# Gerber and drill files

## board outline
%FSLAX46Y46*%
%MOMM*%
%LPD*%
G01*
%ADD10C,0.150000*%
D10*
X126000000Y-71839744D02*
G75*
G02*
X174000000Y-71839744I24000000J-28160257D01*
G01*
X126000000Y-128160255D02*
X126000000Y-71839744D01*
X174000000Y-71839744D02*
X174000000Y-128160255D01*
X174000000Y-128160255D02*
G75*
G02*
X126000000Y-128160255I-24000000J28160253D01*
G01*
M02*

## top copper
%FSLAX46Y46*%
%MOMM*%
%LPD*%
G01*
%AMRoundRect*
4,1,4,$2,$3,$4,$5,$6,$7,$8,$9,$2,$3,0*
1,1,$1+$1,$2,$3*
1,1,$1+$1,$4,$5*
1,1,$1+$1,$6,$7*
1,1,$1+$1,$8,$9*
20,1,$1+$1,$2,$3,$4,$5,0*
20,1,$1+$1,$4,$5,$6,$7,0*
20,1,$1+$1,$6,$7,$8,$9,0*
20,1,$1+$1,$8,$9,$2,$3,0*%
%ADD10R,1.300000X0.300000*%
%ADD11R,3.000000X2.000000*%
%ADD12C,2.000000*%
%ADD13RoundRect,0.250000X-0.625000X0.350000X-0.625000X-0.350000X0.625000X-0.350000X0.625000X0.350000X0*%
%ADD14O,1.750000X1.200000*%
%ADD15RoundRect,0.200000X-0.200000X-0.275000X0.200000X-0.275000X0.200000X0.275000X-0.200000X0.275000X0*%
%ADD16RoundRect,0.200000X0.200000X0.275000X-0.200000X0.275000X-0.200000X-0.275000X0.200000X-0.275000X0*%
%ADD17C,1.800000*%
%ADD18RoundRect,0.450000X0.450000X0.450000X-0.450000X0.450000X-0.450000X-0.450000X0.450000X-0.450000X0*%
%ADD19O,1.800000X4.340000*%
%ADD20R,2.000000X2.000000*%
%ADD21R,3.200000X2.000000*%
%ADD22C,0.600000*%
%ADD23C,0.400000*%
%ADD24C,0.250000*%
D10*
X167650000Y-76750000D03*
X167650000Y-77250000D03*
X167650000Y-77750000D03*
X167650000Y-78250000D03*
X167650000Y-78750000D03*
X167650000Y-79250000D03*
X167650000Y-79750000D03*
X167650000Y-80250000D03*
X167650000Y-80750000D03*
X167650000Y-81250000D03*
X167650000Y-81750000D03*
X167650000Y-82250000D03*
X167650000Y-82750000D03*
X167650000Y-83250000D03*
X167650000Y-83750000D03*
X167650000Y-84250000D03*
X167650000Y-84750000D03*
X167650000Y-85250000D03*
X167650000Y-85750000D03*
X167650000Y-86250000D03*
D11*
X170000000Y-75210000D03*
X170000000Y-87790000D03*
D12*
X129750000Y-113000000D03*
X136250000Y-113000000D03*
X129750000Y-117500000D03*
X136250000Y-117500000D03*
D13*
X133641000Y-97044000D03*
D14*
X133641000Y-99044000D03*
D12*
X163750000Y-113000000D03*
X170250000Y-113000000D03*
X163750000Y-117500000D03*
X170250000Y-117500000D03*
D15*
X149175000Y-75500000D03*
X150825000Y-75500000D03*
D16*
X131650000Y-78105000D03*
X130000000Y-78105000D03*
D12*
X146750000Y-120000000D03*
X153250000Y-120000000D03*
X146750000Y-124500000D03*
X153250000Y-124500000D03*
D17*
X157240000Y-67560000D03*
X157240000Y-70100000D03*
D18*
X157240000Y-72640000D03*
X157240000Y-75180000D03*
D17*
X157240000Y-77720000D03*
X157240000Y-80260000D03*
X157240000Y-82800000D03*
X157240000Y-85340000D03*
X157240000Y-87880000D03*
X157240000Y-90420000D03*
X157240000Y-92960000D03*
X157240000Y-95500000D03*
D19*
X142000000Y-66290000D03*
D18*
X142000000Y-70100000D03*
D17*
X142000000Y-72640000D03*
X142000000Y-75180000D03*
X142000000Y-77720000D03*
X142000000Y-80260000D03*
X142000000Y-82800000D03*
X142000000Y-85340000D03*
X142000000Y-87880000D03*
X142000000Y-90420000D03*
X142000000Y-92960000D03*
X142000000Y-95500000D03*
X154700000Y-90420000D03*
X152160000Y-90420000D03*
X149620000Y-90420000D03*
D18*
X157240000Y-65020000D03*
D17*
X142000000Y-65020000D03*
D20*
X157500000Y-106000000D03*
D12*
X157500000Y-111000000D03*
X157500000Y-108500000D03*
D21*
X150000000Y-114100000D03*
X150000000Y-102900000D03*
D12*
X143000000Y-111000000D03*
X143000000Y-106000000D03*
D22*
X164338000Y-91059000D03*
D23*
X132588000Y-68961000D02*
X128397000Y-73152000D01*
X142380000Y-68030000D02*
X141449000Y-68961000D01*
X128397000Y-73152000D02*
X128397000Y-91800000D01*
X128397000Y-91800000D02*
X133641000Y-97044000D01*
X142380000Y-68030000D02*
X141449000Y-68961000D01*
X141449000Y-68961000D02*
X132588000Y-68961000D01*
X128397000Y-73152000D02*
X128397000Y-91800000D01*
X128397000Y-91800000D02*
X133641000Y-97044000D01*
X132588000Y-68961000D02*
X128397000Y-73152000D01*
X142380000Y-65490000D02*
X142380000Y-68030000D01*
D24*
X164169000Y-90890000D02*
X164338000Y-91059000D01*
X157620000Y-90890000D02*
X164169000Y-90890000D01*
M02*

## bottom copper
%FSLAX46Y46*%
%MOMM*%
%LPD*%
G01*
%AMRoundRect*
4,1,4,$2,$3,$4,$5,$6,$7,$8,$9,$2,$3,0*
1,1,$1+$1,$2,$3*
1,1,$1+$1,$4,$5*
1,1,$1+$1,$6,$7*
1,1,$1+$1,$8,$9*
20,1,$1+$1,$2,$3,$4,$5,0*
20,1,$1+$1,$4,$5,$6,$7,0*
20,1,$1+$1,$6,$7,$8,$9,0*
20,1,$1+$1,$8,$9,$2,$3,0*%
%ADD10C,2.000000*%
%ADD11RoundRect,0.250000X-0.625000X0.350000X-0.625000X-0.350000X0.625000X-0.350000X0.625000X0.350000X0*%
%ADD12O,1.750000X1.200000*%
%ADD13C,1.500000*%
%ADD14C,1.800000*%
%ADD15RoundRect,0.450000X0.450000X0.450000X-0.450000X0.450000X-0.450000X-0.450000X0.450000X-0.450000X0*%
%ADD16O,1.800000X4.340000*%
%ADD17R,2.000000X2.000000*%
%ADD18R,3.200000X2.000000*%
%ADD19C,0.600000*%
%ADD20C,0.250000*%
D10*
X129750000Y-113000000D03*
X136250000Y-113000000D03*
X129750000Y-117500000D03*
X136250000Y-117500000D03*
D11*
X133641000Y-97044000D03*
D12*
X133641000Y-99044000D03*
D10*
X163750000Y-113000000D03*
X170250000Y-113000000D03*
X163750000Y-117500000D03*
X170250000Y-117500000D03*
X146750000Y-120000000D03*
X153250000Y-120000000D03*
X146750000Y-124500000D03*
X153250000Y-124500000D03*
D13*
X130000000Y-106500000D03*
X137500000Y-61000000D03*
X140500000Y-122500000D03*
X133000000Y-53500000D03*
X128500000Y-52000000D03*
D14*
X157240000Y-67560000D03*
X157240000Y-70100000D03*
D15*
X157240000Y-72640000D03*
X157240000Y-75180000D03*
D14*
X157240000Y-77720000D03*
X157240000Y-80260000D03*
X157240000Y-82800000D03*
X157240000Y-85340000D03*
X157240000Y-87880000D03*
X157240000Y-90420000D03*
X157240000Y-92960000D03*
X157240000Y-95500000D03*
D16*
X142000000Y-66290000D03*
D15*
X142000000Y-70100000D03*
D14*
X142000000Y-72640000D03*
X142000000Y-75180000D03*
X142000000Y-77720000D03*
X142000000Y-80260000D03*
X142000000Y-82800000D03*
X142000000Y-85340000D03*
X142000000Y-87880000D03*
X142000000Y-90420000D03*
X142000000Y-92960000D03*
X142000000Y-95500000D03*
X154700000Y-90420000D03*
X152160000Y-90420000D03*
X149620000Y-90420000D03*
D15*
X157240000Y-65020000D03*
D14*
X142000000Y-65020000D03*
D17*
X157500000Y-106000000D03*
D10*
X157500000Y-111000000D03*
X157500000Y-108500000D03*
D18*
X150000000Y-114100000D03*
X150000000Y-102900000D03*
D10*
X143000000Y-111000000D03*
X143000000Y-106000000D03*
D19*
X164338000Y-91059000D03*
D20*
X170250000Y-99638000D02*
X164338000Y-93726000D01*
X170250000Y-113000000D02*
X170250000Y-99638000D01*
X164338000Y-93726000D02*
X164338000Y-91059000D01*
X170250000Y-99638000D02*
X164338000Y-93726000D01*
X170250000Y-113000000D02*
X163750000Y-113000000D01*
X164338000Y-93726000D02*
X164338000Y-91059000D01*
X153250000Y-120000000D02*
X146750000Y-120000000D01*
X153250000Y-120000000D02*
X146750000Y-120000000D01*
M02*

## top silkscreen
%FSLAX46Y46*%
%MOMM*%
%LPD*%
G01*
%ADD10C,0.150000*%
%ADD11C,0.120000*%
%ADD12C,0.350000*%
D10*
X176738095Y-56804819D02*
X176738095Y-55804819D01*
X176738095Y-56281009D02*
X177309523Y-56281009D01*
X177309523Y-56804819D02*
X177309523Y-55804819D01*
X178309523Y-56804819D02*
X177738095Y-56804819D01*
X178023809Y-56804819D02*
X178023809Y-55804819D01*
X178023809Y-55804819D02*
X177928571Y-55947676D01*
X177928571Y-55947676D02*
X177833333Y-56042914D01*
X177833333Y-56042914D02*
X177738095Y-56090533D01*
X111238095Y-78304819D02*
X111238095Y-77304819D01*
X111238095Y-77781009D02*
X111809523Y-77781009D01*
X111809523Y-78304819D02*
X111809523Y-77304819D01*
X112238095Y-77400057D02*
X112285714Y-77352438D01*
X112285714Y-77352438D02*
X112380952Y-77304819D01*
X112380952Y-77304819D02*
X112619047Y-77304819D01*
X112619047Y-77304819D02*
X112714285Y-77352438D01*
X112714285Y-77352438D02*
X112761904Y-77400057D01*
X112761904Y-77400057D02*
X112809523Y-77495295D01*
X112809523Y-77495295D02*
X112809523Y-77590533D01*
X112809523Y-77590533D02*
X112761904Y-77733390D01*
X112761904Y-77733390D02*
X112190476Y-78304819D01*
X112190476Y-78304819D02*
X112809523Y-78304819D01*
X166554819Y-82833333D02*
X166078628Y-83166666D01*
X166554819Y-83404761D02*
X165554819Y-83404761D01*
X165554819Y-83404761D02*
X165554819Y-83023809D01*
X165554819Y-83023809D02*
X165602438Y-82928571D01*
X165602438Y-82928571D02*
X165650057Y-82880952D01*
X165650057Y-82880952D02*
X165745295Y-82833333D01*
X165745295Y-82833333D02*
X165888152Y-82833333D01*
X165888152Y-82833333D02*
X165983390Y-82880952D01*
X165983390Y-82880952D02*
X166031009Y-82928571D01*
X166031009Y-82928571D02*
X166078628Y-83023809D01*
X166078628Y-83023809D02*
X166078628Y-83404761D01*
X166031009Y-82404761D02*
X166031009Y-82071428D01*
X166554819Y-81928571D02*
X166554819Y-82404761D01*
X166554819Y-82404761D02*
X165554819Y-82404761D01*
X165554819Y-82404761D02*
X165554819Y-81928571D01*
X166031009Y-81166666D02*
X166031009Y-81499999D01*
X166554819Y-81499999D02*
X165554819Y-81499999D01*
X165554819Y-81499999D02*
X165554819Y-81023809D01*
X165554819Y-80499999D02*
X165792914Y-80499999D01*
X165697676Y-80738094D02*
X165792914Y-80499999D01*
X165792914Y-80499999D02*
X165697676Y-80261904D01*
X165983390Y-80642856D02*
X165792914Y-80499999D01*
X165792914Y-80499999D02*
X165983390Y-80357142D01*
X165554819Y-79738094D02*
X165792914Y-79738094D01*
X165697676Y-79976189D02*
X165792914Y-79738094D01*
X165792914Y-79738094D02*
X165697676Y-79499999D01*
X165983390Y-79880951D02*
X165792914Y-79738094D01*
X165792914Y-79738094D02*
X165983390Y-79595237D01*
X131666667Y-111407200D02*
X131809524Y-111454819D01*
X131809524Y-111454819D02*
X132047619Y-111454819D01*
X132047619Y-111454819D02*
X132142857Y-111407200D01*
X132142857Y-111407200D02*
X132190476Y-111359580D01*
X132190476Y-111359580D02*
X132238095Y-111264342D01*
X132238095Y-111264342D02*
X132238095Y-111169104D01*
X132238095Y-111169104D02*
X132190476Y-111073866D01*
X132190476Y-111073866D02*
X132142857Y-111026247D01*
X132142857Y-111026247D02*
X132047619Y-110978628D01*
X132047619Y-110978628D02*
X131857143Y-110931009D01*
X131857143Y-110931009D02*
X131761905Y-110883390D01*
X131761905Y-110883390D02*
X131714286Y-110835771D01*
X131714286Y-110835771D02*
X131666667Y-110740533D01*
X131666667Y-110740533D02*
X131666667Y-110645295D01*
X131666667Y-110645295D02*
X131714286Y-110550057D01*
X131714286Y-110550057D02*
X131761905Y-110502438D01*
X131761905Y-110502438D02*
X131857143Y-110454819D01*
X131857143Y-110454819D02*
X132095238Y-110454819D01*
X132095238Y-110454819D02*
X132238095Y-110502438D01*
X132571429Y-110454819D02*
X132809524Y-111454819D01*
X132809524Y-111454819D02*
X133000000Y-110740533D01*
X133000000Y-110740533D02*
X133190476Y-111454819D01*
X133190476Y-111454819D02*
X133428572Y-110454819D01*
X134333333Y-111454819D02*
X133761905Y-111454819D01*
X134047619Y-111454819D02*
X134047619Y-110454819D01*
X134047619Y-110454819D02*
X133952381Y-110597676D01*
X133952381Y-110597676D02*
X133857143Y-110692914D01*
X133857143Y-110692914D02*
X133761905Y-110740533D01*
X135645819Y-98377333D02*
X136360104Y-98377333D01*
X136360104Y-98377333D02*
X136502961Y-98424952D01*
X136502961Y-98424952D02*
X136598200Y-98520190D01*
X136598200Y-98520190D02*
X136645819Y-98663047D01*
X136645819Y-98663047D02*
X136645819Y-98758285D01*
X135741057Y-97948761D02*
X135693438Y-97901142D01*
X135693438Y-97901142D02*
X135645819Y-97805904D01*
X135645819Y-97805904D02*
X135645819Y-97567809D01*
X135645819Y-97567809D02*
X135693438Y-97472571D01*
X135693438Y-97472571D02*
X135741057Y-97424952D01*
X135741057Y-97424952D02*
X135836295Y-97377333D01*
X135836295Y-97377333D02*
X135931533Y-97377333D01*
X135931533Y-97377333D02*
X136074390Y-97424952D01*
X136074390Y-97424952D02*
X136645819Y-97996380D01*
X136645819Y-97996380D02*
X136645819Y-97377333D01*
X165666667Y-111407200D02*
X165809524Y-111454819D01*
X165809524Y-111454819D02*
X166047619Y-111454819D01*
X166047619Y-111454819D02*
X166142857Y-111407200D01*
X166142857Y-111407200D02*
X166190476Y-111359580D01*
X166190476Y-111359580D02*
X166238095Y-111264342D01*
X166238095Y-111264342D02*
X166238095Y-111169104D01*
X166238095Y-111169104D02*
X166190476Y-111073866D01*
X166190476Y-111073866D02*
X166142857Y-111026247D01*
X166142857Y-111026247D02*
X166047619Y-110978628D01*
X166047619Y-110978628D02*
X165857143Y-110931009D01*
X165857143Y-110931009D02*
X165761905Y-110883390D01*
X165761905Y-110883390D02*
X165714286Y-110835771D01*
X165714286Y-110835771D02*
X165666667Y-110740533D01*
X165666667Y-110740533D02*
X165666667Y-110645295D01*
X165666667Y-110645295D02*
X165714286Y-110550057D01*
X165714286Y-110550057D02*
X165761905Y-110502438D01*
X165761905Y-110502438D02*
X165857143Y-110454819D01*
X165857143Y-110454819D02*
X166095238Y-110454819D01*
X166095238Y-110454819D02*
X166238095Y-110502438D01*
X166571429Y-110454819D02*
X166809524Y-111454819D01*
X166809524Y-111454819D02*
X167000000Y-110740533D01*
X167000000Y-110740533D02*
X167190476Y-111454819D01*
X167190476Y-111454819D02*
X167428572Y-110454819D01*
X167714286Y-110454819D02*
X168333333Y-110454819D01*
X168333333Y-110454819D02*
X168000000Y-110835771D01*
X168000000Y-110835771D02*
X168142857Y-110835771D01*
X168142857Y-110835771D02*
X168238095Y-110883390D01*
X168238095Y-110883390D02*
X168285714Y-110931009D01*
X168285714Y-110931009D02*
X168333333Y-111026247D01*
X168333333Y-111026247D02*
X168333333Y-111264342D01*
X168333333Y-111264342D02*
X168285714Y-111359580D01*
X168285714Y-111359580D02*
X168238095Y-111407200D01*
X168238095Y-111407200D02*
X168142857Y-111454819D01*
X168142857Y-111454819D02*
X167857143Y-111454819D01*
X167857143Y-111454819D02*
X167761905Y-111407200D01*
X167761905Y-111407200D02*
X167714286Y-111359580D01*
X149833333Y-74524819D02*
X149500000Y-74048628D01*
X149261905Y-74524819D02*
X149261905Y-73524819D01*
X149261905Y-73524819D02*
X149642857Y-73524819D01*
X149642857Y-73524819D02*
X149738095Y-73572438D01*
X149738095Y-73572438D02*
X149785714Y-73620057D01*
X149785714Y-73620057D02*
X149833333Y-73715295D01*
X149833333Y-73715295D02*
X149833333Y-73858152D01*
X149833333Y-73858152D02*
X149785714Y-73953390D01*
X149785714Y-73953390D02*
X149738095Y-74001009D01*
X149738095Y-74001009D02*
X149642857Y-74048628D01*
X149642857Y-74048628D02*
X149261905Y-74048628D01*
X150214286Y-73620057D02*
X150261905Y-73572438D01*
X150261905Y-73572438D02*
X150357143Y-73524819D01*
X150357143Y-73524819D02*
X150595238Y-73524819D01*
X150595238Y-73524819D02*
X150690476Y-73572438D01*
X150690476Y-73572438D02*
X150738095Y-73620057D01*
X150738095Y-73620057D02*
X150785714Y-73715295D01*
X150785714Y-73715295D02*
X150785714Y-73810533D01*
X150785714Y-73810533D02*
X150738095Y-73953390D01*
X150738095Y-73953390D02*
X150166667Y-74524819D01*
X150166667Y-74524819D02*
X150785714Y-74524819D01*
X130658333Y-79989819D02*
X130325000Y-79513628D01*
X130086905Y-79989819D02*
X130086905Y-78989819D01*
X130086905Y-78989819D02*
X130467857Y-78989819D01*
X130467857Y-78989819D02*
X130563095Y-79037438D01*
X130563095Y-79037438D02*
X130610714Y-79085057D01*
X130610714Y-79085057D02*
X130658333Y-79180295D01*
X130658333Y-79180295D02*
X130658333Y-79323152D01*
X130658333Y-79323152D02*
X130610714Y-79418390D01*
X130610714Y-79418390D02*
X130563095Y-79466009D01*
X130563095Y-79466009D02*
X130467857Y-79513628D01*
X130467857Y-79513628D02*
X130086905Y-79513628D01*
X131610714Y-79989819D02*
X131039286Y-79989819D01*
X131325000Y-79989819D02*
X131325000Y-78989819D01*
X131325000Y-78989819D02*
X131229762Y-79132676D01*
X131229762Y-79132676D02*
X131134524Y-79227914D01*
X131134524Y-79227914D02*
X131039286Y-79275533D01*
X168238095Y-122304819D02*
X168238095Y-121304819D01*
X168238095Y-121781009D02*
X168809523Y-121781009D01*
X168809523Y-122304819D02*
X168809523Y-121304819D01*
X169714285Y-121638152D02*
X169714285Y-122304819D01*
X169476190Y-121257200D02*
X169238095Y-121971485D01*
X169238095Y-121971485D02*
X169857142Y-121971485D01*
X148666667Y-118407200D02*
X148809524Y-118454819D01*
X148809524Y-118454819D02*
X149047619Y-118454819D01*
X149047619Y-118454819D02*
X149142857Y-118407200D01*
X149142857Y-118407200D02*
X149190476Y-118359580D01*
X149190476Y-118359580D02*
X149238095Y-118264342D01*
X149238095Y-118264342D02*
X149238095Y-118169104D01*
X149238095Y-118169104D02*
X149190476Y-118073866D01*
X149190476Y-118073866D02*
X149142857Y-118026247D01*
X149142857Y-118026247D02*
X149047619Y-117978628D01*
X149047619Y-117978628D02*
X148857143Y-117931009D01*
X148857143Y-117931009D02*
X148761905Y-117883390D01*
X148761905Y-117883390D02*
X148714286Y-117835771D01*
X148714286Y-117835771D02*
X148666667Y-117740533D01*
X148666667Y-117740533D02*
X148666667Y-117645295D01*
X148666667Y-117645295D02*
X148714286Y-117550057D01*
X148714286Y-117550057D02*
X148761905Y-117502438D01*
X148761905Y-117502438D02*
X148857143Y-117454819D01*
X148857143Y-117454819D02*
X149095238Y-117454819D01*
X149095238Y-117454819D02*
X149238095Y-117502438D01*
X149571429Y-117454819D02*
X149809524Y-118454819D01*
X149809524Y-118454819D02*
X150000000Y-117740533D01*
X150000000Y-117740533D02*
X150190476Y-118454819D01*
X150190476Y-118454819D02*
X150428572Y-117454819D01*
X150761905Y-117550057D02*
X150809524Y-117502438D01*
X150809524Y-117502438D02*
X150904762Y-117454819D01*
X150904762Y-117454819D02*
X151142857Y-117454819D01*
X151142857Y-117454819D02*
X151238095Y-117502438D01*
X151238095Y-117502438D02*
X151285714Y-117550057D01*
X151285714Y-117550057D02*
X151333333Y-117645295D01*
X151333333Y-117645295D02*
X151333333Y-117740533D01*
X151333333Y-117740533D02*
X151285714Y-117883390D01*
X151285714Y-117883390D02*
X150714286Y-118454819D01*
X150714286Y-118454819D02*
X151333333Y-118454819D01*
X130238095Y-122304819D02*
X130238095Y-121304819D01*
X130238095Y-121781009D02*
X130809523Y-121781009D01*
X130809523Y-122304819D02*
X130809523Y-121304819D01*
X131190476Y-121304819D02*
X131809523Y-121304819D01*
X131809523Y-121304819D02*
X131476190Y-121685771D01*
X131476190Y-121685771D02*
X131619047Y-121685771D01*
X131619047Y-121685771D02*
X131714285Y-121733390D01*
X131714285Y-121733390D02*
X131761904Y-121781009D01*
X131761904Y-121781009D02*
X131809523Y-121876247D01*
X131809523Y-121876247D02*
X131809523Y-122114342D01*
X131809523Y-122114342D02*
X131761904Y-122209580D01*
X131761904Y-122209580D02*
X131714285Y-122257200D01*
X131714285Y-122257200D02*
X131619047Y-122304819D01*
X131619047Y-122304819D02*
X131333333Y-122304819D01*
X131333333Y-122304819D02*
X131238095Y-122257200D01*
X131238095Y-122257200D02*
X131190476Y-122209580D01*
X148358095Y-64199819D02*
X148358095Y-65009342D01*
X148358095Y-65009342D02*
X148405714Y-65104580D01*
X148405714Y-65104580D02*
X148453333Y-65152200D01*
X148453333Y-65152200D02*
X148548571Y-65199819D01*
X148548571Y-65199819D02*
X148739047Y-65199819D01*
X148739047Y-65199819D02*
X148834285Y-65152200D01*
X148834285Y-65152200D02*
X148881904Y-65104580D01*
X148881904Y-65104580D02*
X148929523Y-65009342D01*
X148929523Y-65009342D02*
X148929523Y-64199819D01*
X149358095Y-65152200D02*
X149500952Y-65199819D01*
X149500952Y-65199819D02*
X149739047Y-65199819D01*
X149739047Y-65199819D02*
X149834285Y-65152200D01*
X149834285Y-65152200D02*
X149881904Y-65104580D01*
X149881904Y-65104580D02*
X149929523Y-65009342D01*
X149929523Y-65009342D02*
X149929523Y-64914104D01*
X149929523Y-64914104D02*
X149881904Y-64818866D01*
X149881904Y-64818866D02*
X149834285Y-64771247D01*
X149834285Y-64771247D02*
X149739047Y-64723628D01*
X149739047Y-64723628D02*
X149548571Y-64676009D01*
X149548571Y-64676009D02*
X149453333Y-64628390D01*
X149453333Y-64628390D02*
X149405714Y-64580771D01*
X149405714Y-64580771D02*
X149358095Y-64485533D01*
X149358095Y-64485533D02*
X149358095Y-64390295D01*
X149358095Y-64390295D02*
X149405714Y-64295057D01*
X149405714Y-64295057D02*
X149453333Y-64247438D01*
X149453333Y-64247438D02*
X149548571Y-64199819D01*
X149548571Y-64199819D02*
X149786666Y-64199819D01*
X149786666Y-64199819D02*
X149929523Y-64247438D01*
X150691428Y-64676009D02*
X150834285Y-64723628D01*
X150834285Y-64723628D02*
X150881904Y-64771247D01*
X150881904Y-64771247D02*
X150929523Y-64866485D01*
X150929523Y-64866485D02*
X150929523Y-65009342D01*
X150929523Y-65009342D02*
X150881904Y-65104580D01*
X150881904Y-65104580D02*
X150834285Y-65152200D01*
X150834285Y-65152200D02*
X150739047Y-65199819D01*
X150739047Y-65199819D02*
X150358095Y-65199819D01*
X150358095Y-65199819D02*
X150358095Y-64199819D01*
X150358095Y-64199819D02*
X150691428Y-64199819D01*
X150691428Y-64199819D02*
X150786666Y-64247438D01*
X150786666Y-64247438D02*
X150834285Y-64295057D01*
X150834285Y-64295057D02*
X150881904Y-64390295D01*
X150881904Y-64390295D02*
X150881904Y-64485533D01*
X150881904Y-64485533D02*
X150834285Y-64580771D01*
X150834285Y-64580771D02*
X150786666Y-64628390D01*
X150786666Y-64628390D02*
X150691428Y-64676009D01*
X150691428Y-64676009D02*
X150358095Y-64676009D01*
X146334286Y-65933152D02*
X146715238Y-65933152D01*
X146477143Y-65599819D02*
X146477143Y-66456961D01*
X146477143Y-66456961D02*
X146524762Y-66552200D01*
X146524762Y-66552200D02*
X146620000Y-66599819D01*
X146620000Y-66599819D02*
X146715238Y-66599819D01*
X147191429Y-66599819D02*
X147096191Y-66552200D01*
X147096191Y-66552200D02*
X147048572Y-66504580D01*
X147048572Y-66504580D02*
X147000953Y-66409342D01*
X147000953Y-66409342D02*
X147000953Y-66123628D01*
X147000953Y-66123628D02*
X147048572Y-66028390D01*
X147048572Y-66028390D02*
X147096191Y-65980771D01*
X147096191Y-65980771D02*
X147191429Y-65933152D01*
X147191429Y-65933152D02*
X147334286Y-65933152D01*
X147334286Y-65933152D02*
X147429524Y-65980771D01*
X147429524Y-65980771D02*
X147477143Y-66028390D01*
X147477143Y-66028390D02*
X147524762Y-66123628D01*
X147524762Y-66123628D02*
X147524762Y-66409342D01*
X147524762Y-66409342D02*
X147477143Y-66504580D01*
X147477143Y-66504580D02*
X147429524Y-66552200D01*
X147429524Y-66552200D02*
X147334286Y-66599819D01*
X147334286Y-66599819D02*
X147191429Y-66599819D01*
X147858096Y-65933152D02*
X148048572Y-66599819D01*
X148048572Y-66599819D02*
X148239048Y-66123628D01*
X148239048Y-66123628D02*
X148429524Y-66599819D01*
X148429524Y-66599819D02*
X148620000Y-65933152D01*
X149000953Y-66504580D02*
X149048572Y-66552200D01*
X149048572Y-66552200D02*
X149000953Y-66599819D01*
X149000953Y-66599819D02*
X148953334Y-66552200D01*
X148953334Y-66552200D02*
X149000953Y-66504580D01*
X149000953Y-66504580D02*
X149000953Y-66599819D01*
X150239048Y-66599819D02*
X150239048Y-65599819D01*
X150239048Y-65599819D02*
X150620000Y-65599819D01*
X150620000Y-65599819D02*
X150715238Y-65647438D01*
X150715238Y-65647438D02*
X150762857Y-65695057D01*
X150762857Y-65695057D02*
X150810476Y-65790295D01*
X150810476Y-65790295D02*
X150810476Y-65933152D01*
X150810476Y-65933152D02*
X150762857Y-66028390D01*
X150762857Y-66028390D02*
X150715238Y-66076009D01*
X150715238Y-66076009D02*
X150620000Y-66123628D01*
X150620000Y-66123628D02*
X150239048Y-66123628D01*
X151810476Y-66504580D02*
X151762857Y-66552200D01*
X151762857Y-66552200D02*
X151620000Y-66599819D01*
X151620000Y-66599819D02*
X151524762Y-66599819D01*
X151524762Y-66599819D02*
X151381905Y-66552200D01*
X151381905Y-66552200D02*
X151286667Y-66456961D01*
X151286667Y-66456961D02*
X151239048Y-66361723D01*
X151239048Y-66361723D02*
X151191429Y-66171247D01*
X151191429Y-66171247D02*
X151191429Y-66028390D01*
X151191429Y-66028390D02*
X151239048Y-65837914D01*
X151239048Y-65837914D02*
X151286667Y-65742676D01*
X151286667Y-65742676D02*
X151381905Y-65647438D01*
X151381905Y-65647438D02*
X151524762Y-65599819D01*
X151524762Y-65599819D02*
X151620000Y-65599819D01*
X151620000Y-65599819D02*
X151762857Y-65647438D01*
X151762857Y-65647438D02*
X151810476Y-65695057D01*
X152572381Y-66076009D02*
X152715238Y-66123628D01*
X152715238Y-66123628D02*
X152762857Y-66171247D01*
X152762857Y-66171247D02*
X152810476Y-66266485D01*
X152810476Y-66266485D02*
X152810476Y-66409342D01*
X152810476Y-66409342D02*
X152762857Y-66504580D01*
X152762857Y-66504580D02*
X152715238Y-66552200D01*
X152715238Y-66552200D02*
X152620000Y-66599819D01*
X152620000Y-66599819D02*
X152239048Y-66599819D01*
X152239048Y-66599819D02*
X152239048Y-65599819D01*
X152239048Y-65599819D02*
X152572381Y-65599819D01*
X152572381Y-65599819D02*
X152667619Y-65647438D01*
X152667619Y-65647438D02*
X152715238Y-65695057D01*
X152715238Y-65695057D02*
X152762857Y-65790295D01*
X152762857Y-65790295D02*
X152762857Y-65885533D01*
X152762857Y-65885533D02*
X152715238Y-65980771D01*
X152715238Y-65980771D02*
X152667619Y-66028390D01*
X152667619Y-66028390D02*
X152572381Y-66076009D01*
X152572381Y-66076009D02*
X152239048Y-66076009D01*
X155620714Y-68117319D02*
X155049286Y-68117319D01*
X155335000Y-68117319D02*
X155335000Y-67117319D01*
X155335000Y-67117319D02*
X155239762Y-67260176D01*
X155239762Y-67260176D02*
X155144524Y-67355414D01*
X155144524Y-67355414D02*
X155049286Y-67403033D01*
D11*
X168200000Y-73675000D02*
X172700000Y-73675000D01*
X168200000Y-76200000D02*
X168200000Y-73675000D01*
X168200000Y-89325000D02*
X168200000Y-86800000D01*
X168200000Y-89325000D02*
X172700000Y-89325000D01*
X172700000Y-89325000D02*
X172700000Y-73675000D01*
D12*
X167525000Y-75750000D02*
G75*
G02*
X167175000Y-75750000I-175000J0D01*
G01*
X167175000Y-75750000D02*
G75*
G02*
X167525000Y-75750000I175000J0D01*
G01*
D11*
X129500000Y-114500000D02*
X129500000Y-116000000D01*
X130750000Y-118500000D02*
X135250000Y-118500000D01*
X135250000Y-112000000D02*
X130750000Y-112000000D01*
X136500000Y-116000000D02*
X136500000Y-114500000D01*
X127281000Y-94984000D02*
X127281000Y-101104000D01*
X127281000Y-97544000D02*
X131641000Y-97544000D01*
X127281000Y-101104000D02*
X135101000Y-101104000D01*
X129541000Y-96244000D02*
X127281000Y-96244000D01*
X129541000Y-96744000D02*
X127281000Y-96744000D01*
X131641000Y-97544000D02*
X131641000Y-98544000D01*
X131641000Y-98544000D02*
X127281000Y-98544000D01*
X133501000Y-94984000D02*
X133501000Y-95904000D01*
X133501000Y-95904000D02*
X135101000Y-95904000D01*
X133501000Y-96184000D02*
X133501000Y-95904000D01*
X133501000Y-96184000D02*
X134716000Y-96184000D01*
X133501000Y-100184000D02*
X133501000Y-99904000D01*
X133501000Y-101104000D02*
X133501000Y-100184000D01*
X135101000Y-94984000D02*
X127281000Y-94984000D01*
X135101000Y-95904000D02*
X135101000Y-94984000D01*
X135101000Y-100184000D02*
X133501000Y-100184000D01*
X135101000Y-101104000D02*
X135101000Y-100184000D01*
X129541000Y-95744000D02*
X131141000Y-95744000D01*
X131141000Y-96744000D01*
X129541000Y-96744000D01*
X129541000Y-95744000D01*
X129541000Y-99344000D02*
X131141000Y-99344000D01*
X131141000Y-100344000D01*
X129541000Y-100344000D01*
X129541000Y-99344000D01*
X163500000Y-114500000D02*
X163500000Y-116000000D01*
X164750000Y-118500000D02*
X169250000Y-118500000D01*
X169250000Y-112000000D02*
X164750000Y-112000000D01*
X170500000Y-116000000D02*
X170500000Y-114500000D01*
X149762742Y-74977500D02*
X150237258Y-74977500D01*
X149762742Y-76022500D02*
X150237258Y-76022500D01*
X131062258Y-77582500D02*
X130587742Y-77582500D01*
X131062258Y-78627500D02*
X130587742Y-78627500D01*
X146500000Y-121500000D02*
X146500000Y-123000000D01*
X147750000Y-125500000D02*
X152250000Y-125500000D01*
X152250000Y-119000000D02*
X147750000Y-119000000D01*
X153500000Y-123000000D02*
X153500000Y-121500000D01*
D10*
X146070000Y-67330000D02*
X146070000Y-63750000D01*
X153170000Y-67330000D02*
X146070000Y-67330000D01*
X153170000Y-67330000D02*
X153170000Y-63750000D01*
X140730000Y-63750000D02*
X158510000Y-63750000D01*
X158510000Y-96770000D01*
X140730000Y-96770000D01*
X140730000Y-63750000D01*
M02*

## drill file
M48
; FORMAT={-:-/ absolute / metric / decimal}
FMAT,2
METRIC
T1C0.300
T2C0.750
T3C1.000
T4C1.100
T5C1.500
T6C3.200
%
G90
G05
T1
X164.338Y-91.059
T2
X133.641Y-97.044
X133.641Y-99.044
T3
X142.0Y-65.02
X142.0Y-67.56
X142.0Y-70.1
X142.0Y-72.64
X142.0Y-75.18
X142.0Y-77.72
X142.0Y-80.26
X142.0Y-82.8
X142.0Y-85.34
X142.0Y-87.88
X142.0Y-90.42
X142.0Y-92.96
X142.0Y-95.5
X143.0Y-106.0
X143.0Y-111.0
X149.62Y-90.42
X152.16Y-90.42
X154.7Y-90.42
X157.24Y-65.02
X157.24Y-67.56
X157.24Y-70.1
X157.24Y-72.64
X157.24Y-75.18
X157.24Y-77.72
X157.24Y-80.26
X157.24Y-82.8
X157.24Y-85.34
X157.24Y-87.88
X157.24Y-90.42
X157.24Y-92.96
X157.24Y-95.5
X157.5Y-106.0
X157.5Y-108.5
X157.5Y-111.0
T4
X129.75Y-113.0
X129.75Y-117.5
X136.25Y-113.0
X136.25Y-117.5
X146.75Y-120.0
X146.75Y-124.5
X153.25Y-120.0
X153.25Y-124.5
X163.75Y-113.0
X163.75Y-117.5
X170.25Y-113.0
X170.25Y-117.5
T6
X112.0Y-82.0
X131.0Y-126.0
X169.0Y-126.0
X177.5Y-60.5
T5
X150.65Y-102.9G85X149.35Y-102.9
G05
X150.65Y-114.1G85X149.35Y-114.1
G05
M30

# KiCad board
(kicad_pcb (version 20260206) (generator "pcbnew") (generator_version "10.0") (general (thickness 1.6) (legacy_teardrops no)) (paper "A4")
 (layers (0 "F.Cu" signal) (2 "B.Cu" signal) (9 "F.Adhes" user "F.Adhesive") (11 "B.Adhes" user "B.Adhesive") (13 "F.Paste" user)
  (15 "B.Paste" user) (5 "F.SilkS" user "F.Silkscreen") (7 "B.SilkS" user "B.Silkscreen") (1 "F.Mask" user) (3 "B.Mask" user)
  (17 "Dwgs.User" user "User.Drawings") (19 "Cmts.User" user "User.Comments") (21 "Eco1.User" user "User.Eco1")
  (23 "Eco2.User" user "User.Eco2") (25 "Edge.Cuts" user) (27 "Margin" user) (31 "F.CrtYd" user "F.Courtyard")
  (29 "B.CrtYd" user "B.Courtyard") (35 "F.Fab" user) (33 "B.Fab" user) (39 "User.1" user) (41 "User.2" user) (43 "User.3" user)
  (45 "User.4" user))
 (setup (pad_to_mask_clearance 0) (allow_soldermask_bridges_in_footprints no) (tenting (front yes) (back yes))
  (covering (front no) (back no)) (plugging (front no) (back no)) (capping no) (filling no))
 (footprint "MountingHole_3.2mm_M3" (layer "F.Cu") (at 177.5 60.5)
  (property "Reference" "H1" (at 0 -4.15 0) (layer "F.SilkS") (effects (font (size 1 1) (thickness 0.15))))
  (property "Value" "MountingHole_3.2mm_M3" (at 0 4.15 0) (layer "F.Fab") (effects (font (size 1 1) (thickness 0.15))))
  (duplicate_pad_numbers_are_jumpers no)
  (pad "" np_thru_hole circle (at 0 0) (size 3.2 3.2) (drill 3.2) (layers "*.Cu" "*.Mask")))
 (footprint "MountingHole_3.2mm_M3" (layer "F.Cu") (at 112 82)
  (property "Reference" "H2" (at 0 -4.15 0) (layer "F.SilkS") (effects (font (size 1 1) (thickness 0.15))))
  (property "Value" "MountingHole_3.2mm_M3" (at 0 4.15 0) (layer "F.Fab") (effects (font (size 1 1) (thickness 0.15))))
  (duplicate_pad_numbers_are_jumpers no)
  (pad "" np_thru_hole circle (at 0 0) (size 3.2 3.2) (drill 3.2) (layers "*.Cu" "*.Mask")))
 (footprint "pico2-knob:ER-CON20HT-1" (layer "F.Cu") (at 169.5 81.5 -90)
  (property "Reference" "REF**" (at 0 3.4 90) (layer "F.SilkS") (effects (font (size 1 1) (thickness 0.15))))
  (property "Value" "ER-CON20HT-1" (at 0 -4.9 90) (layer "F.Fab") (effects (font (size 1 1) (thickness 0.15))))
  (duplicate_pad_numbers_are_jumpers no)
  (fp_line (start -7.825 1.3) (end -7.825 -3.2) (stroke (width 0.12) (type solid)) (layer "F.SilkS"))
  (fp_line (start -5.3 1.3) (end -7.825 1.3) (stroke (width 0.12) (type solid)) (layer "F.SilkS"))
  (fp_line (start 7.825 1.3) (end 5.3 1.3) (stroke (width 0.12) (type solid)) (layer "F.SilkS"))
  (fp_line (start 7.825 1.3) (end 7.825 -3.2) (stroke (width 0.12) (type solid)) (layer "F.SilkS"))
  (fp_line (start 7.825 -3.2) (end -7.825 -3.2) (stroke (width 0.12) (type solid)) (layer "F.SilkS"))
  (fp_circle (center -5.75 2.15) (end -5.55 2.15) (stroke (width 0.3) (type solid)) (fill yes) (layer "F.SilkS"))
  (pad "1" smd rect (at -4.75 1.85 270) (size 0.3 1.3) (layers "F.Cu" "F.Mask" "F.Paste"))
  (pad "2" smd rect (at -4.25 1.85 270) (size 0.3 1.3) (layers "F.Cu" "F.Mask" "F.Paste"))
  (pad "3" smd rect (at -3.75 1.85 270) (size 0.3 1.3) (layers "F.Cu" "F.Mask" "F.Paste"))
  (pad "4" smd rect (at -3.25 1.85 270) (size 0.3 1.3) (layers "F.Cu" "F.Mask" "F.Paste"))
  (pad "5" smd rect (at -2.75 1.85 270) (size 0.3 1.3) (layers "F.Cu" "F.Mask" "F.Paste"))
  (pad "6" smd rect (at -2.25 1.85 270) (size 0.3 1.3) (layers "F.Cu" "F.Mask" "F.Paste"))
  (pad "7" smd rect (at -1.75 1.85 270) (size 0.3 1.3) (layers "F.Cu" "F.Mask" "F.Paste"))
  (pad "8" smd rect (at -1.25 1.85 270) (size 0.3 1.3) (layers "F.Cu" "F.Mask" "F.Paste"))
  (pad "9" smd rect (at -0.75 1.85 270) (size 0.3 1.3) (layers "F.Cu" "F.Mask" "F.Paste"))
  (pad "10" smd rect (at -0.25 1.85 270) (size 0.3 1.3) (layers "F.Cu" "F.Mask" "F.Paste"))
  (pad "11" smd rect (at 0.25 1.85 270) (size 0.3 1.3) (layers "F.Cu" "F.Mask" "F.Paste"))
  (pad "12" smd rect (at 0.75 1.85 270) (size 0.3 1.3) (layers "F.Cu" "F.Mask" "F.Paste"))
  (pad "13" smd rect (at 1.25 1.85 270) (size 0.3 1.3) (layers "F.Cu" "F.Mask" "F.Paste"))
  (pad "14" smd rect (at 1.75 1.85 270) (size 0.3 1.3) (layers "F.Cu" "F.Mask" "F.Paste"))
  (pad "15" smd rect (at 2.25 1.85 270) (size 0.3 1.3) (layers "F.Cu" "F.Mask" "F.Paste"))
  (pad "16" smd rect (at 2.75 1.85 270) (size 0.3 1.3) (layers "F.Cu" "F.Mask" "F.Paste"))
  (pad "17" smd rect (at 3.25 1.85 270) (size 0.3 1.3) (layers "F.Cu" "F.Mask" "F.Paste"))
  (pad "18" smd rect (at 3.75 1.85 270) (size 0.3 1.3) (layers "F.Cu" "F.Mask" "F.Paste"))
  (pad "19" smd rect (at 4.25 1.85 270) (size 0.3 1.3) (layers "F.Cu" "F.Mask" "F.Paste"))
  (pad "20" smd rect (at 4.75 1.85 270) (size 0.3 1.3) (layers "F.Cu" "F.Mask" "F.Paste"))
  (pad "MP" smd rect (at -6.29 -0.5 270) (size 2 3) (layers "F.Cu" "F.Mask" "F.Paste"))
  (pad "MP" smd rect (at 6.29 -0.5 270) (size 2 3) (layers "F.Cu" "F.Mask" "F.Paste")))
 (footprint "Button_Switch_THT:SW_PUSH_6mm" (layer "F.Cu") (at 129.75 113)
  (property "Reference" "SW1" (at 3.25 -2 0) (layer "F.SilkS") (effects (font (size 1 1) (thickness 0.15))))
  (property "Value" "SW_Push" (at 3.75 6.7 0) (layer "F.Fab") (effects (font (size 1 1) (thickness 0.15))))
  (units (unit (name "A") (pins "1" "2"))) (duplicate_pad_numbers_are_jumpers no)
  (fp_line (start -0.25 1.5) (end -0.25 3) (stroke (width 0.12) (type solid)) (layer "F.SilkS"))
  (fp_line (start 1 5.5) (end 5.5 5.5) (stroke (width 0.12) (type solid)) (layer "F.SilkS"))
  (fp_line (start 5.5 -1) (end 1 -1) (stroke (width 0.12) (type solid)) (layer "F.SilkS"))
  (fp_line (start 6.75 3) (end 6.75 1.5) (stroke (width 0.12) (type solid)) (layer "F.SilkS"))
  (pad "1" thru_hole circle (at 0 0 90) (size 2 2) (drill 1.1) (layers "*.Cu" "*.Mask") (remove_unused_layers no) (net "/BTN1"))
  (pad "1" thru_hole circle (at 6.5 0 90) (size 2 2) (drill 1.1) (layers "*.Cu" "*.Mask") (remove_unused_layers no) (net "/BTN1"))
  (pad "2" thru_hole circle (at 0 4.5 90) (size 2 2) (drill 1.1) (layers "*.Cu" "*.Mask") (remove_unused_layers no) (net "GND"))
  (pad "2" thru_hole circle (at 6.5 4.5 90) (size 2 2) (drill 1.1) (layers "*.Cu" "*.Mask") (remove_unused_layers no) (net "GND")))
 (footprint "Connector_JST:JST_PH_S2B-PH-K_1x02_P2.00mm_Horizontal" (layer "F.Cu") (at 133.641 97.044 -90)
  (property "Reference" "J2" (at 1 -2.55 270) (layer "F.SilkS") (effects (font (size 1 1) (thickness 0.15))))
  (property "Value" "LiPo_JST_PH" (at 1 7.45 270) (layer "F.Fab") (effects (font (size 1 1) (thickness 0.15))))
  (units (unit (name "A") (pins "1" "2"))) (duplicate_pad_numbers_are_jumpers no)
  (fp_line (start -2.06 6.36) (end 4.06 6.36) (stroke (width 0.12) (type solid)) (layer "F.SilkS"))
  (fp_line (start 0.5 6.36) (end 0.5 2) (stroke (width 0.12) (type solid)) (layer "F.SilkS"))
  (fp_line (start 4.06 6.36) (end 4.06 -1.46) (stroke (width 0.12) (type solid)) (layer "F.SilkS"))
  (fp_line (start -0.8 4.1) (end -0.8 6.36) (stroke (width 0.12) (type solid)) (layer "F.SilkS"))
  (fp_line (start -0.3 4.1) (end -0.3 6.36) (stroke (width 0.12) (type solid)) (layer "F.SilkS"))
  (fp_line (start 0.5 2) (end 1.5 2) (stroke (width 0.12) (type solid)) (layer "F.SilkS"))
  (fp_line (start 1.5 2) (end 1.5 6.36) (stroke (width 0.12) (type solid)) (layer "F.SilkS"))
  (fp_line (start -2.06 0.14) (end -1.14 0.14) (stroke (width 0.12) (type solid)) (layer "F.SilkS"))
  (fp_line (start -1.14 0.14) (end -1.14 -1.46) (stroke (width 0.12) (type solid)) (layer "F.SilkS"))
  (fp_line (start -0.86 0.14) (end -1.14 0.14) (stroke (width 0.12) (type solid)) (layer "F.SilkS"))
  (fp_line (start -0.86 0.14) (end -0.86 -1.075) (stroke (width 0.12) (type solid)) (layer "F.SilkS"))
  (fp_line (start 3.14 0.14) (end 2.86 0.14) (stroke (width 0.12) (type solid)) (layer "F.SilkS"))
  (fp_line (start 4.06 0.14) (end 3.14 0.14) (stroke (width 0.12) (type solid)) (layer "F.SilkS"))
  (fp_line (start -2.06 -1.46) (end -2.06 6.36) (stroke (width 0.12) (type solid)) (layer "F.SilkS"))
  (fp_line (start -1.14 -1.46) (end -2.06 -1.46) (stroke (width 0.12) (type solid)) (layer "F.SilkS"))
  (fp_line (start 3.14 -1.46) (end 3.14 0.14) (stroke (width 0.12) (type solid)) (layer "F.SilkS"))
  (fp_line (start 4.06 -1.46) (end 3.14 -1.46) (stroke (width 0.12) (type solid)) (layer "F.SilkS"))
  (fp_rect (start -1.3 2.5) (end -0.3 4.1) (stroke (width 0.12) (type solid)) (fill no) (layer "F.SilkS"))
  (fp_rect (start 2.3 2.5) (end 3.3 4.1) (stroke (width 0.12) (type solid)) (fill no) (layer "F.SilkS"))
  (pad "1" thru_hole roundrect (at 0 0 270) (size 1.2 1.75) (drill 0.75) (layers "*.Cu" "*.Mask") (remove_unused_layers no)
   (roundrect_rratio 0.208333) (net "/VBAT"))
  (pad "2" thru_hole oval (at 2 0 270) (size 1.2 1.75) (drill 0.75) (layers "*.Cu" "*.Mask") (remove_unused_layers no) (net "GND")
   (zone_connect 2)))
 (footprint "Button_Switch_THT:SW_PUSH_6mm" (layer "F.Cu") (at 163.75 113)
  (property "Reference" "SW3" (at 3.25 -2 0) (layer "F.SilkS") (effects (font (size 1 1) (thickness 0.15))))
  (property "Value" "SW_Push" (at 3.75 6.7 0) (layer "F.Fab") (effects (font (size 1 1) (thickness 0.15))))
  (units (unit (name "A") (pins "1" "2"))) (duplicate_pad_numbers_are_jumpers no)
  (fp_line (start -0.25 1.5) (end -0.25 3) (stroke (width 0.12) (type solid)) (layer "F.SilkS"))
  (fp_line (start 1 5.5) (end 5.5 5.5) (stroke (width 0.12) (type solid)) (layer "F.SilkS"))
  (fp_line (start 5.5 -1) (end 1 -1) (stroke (width 0.12) (type solid)) (layer "F.SilkS"))
  (fp_line (start 6.75 3) (end 6.75 1.5) (stroke (width 0.12) (type solid)) (layer "F.SilkS"))
  (pad "1" thru_hole circle (at 0 0 90) (size 2 2) (drill 1.1) (layers "*.Cu" "*.Mask") (remove_unused_layers no) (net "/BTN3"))
  (pad "1" thru_hole circle (at 6.5 0 90) (size 2 2) (drill 1.1) (layers "*.Cu" "*.Mask") (remove_unused_layers no) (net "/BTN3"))
  (pad "2" thru_hole circle (at 0 4.5 90) (size 2 2) (drill 1.1) (layers "*.Cu" "*.Mask") (remove_unused_layers no) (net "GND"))
  (pad "2" thru_hole circle (at 6.5 4.5 90) (size 2 2) (drill 1.1) (layers "*.Cu" "*.Mask") (remove_unused_layers no) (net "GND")))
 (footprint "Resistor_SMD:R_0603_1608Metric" (layer "F.Cu") (at 150 75.5)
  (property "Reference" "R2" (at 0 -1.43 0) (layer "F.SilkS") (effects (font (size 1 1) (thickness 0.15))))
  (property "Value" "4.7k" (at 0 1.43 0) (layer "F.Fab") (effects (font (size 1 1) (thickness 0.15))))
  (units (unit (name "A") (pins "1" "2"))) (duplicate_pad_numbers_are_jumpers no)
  (fp_line (start -0.237258 -0.5225) (end 0.237258 -0.5225) (stroke (width 0.12) (type solid)) (layer "F.SilkS"))
  (fp_line (start -0.237258 0.5225) (end 0.237258 0.5225) (stroke (width 0.12) (type solid)) (layer "F.SilkS"))
  (pad "1" smd roundrect (at -0.825 0) (size 0.8 0.95) (layers "F.Cu" "F.Mask" "F.Paste") (roundrect_rratio 0.25) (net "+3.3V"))
  (pad "2" smd roundrect (at 0.825 0) (size 0.8 0.95) (layers "F.Cu" "F.Mask" "F.Paste") (roundrect_rratio 0.25) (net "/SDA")))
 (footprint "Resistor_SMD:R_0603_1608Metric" (layer "F.Cu") (at 130.825 78.105 180)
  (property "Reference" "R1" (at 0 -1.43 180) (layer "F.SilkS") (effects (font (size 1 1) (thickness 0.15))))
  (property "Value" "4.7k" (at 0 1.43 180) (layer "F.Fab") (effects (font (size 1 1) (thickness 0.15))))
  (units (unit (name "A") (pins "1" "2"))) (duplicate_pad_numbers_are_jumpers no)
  (fp_line (start -0.237258 0.5225) (end 0.237258 0.5225) (stroke (width 0.12) (type solid)) (layer "F.SilkS"))
  (fp_line (start -0.237258 -0.5225) (end 0.237258 -0.5225) (stroke (width 0.12) (type solid)) (layer "F.SilkS"))
  (pad "1" smd roundrect (at -0.825 0 180) (size 0.8 0.95) (layers "F.Cu" "F.Mask" "F.Paste") (roundrect_rratio 0.25) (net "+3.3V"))
  (pad "2" smd roundrect (at 0.825 0 180) (size 0.8 0.95) (layers "F.Cu" "F.Mask" "F.Paste") (roundrect_rratio 0.25) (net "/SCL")))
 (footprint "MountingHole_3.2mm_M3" (layer "F.Cu") (at 169 126)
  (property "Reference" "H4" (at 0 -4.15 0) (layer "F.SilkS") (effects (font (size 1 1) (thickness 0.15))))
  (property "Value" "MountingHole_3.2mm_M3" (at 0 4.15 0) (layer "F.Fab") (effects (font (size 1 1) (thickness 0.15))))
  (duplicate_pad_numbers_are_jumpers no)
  (pad "" np_thru_hole circle (at 0 0) (size 3.2 3.2) (drill 3.2) (layers "*.Cu" "*.Mask")))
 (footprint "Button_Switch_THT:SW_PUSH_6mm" (layer "F.Cu") (at 146.75 120)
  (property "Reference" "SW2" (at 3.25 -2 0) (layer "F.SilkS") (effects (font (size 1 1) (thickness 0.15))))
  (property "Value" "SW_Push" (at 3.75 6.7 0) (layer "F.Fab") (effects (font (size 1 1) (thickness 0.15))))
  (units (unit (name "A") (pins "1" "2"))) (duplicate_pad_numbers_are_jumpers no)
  (fp_line (start -0.25 1.5) (end -0.25 3) (stroke (width 0.12) (type solid)) (layer "F.SilkS"))
  (fp_line (start 1 5.5) (end 5.5 5.5) (stroke (width 0.12) (type solid)) (layer "F.SilkS"))
  (fp_line (start 5.5 -1) (end 1 -1) (stroke (width 0.12) (type solid)) (layer "F.SilkS"))
  (fp_line (start 6.75 3) (end 6.75 1.5) (stroke (width 0.12) (type solid)) (layer "F.SilkS"))
  (pad "1" thru_hole circle (at 0 0 90) (size 2 2) (drill 1.1) (layers "*.Cu" "*.Mask") (remove_unused_layers no) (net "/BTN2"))
  (pad "1" thru_hole circle (at 6.5 0 90) (size 2 2) (drill 1.1) (layers "*.Cu" "*.Mask") (remove_unused_layers no) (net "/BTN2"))
  (pad "2" thru_hole circle (at 0 4.5 90) (size 2 2) (drill 1.1) (layers "*.Cu" "*.Mask") (remove_unused_layers no) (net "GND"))
  (pad "2" thru_hole circle (at 6.5 4.5 90) (size 2 2) (drill 1.1) (layers "*.Cu" "*.Mask") (remove_unused_layers no) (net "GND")))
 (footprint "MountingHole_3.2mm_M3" (layer "F.Cu") (at 131 126)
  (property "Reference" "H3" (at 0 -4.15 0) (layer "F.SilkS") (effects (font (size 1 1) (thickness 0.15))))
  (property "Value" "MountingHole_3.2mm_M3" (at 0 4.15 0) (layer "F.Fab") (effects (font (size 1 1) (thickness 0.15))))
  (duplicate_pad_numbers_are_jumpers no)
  (pad "" np_thru_hole circle (at 0 0) (size 3.2 3.2) (drill 3.2) (layers "*.Cu" "*.Mask")))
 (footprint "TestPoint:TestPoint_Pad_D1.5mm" (layer "B.Cu") (at 130 106.5 180)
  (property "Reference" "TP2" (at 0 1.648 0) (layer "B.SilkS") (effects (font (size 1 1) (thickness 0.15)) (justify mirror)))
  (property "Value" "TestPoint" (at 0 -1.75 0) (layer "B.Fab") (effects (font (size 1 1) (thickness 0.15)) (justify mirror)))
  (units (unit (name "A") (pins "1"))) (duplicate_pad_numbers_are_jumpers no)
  (pad "1" smd circle (at 0 0 180) (size 1.5 1.5) (layers "B.Cu" "B.Mask") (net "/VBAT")))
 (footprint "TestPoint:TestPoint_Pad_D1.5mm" (layer "B.Cu") (at 137.5 61 180)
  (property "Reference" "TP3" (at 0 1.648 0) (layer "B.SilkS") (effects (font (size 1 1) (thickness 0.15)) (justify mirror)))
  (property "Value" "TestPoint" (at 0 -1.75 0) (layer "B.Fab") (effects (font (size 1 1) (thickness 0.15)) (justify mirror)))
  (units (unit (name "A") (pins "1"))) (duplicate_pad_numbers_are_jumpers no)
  (pad "1" smd circle (at 0 0 180) (size 1.5 1.5) (layers "B.Cu" "B.Mask") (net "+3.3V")))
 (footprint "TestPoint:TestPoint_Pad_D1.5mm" (layer "B.Cu") (at 140.5 122.5 180)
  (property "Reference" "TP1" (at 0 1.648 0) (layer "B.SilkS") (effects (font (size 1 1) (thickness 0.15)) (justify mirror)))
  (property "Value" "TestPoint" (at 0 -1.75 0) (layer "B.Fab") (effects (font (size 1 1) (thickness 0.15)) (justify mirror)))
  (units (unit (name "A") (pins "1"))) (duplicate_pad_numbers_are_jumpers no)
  (pad "1" smd circle (at 0 0 180) (size 1.5 1.5) (layers "B.Cu" "B.Mask") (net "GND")))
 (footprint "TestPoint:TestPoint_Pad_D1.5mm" (layer "B.Cu") (at 133 53.5 180)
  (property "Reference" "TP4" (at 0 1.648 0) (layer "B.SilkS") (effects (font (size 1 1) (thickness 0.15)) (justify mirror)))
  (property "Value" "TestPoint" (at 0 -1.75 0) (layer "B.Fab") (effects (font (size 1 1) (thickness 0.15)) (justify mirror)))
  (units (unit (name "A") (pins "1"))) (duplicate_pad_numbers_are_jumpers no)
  (pad "1" smd circle (at 0 0 180) (size 1.5 1.5) (layers "B.Cu" "B.Mask") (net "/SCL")))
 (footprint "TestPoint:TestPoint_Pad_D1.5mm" (layer "B.Cu") (at 128.5 52 180)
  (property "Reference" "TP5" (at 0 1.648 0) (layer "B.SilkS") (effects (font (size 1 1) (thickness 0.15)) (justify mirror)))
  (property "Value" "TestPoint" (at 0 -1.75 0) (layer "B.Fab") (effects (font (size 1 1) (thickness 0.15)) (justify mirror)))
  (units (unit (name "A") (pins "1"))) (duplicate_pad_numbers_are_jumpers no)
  (pad "1" smd circle (at 0 0 180) (size 1.5 1.5) (layers "B.Cu" "B.Mask") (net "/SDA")))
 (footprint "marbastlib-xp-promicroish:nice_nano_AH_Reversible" (layer "B.Cu") (at 149.62 81.53 180)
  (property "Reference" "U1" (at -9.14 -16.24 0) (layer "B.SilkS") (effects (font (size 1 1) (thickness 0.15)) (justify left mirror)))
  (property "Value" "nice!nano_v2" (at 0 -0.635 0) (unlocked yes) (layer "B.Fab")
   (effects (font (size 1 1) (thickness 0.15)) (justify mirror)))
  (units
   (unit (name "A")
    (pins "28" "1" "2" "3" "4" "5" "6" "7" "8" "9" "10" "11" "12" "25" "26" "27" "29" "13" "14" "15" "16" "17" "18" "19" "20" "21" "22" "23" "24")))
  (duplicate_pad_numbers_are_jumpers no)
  (fp_line (start 3.55 14.2) (end 3.55 17.78) (stroke (width 0.15) (type default)) (layer "F.SilkS"))
  (fp_line (start -3.55 14.2) (end 3.55 14.2) (stroke (width 0.15) (type default)) (layer "F.SilkS"))
  (fp_line (start -3.55 14.2) (end -3.55 17.78) (stroke (width 0.15) (type default)) (layer "F.SilkS"))
  (fp_rect (start 8.89 17.78) (end -8.89 -15.24) (stroke (width 0.15) (type solid)) (fill no) (layer "F.SilkS"))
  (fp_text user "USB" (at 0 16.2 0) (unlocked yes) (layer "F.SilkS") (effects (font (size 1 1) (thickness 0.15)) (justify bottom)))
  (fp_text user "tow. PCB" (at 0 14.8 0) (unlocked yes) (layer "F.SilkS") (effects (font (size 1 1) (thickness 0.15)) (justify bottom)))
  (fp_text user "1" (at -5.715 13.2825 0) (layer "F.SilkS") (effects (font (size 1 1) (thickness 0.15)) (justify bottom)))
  (pad "1" thru_hole circle (at -7.62 13.97 180) (size 1.8 1.8) (drill 1) (layers "*.Cu" "*.Mask") (remove_unused_layers no)
   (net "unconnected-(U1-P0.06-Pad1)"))
  (pad "2" thru_hole circle (at -7.62 11.43 180) (size 1.8 1.8) (drill 1) (layers "*.Cu" "*.Mask") (remove_unused_layers no)
   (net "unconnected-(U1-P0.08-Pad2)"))
  (pad "3" thru_hole roundrect (at -7.62 8.89 180) (size 1.8 1.8) (drill 1) (layers "*.Cu" "*.Mask") (remove_unused_layers no)
   (roundrect_rratio 0.25) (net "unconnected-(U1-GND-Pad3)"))
  (pad "4" thru_hole roundrect (at -7.62 6.35 180) (size 1.8 1.8) (drill 1) (layers "*.Cu" "*.Mask") (remove_unused_layers no)
   (roundrect_rratio 0.25) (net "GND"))
  (pad "5" thru_hole circle (at -7.62 3.81 180) (size 1.8 1.8) (drill 1) (layers "*.Cu" "*.Mask") (remove_unused_layers no) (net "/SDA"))
  (pad "6" thru_hole circle (at -7.62 1.27 180) (size 1.8 1.8) (drill 1) (layers "*.Cu" "*.Mask") (remove_unused_layers no) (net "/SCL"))
  (pad "7" thru_hole circle (at -7.62 -1.27 180) (size 1.8 1.8) (drill 1) (layers "*.Cu" "*.Mask") (remove_unused_layers no)
   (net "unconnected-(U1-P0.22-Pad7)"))
  (pad "8" thru_hole circle (at -7.62 -3.81 180) (size 1.8 1.8) (drill 1) (layers "*.Cu" "*.Mask") (remove_unused_layers no) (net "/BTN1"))
  (pad "9" thru_hole circle (at -7.62 -6.35 180) (size 1.8 1.8) (drill 1) (layers "*.Cu" "*.Mask") (remove_unused_layers no) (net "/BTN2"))
  (pad "10" thru_hole circle (at -7.62 -8.89 180) (size 1.8 1.8) (drill 1) (layers "*.Cu" "*.Mask") (remove_unused_layers no) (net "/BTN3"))
  (pad "11" thru_hole circle (at -7.62 -11.43 180) (size 1.8 1.8) (drill 1) (layers "*.Cu" "*.Mask") (remove_unused_layers no)
   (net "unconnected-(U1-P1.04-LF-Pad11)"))
  (pad "12" thru_hole circle (at -7.62 -13.97 180) (size 1.8 1.8) (drill 1) (layers "*.Cu" "*.Mask") (remove_unused_layers no)
   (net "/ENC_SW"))
  (pad "13" thru_hole oval (at 7.62 13.97 180) (size 1.8 4.34) (drill 1 (offset 0 1.27)) (layers "*.Cu" "*.Mask") (remove_unused_layers no)
   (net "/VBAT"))
  (pad "14" thru_hole roundrect (at 7.62 11.43 180) (size 1.8 1.8) (drill 1) (layers "*.Cu" "*.Mask") (remove_unused_layers no)
   (roundrect_rratio 0.25) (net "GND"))
  (pad "15" thru_hole circle (at 7.62 8.89 180) (size 1.8 1.8) (drill 1) (layers "*.Cu" "*.Mask") (remove_unused_layers no)
   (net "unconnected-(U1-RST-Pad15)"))
  (pad "16" thru_hole circle (at 7.62 6.35 180) (size 1.8 1.8) (drill 1) (layers "*.Cu" "*.Mask") (remove_unused_layers no) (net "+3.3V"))
  (pad "17" thru_hole circle (at 7.62 3.81 180) (size 1.8 1.8) (drill 1) (layers "*.Cu" "*.Mask") (remove_unused_layers no)
   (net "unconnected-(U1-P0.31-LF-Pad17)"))
  (pad "18" thru_hole circle (at 7.62 1.27 180) (size 1.8 1.8) (drill 1) (layers "*.Cu" "*.Mask") (remove_unused_layers no)
   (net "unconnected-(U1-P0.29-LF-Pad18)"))
  (pad "19" thru_hole circle (at 7.62 -1.27 180) (size 1.8 1.8) (drill 1) (layers "*.Cu" "*.Mask") (remove_unused_layers no)
   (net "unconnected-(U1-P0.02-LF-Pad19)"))
  (pad "20" thru_hole circle (at 7.62 -3.81 180) (size 1.8 1.8) (drill 1) (layers "*.Cu" "*.Mask") (remove_unused_layers no)
   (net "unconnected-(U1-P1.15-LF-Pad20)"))
  (pad "21" thru_hole circle (at 7.62 -6.35 180) (size 1.8 1.8) (drill 1) (layers "*.Cu" "*.Mask") (remove_unused_layers no)
   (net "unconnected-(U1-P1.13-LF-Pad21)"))
  (pad "22" thru_hole circle (at 7.62 -8.89 180) (size 1.8 1.8) (drill 1) (layers "*.Cu" "*.Mask") (remove_unused_layers no)
   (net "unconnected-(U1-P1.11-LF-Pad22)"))
  (pad "23" thru_hole circle (at 7.62 -11.43 180) (size 1.8 1.8) (drill 1) (layers "*.Cu" "*.Mask") (remove_unused_layers no) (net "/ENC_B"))
  (pad "24" thru_hole circle (at 7.62 -13.97 180) (size 1.8 1.8) (drill 1) (layers "*.Cu" "*.Mask") (remove_unused_layers no) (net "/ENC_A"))
  (pad "25" thru_hole circle (at -5.08 -8.89 180) (size 1.8 1.8) (drill 1) (layers "*.Cu" "*.Mask") (remove_unused_layers no)
   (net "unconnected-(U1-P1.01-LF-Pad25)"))
  (pad "26" thru_hole circle (at -2.54 -8.89 180) (size 1.8 1.8) (drill 1) (layers "*.Cu" "*.Mask") (remove_unused_layers no)
   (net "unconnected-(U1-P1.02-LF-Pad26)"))
  (pad "27" thru_hole circle (at 0 -8.89 180) (size 1.8 1.8) (drill 1) (layers "*.Cu" "*.Mask") (remove_unused_layers no)
   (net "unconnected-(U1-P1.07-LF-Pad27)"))
  (pad "28" thru_hole roundrect (at -7.62 16.51 180) (size 1.8 1.8) (drill 1) (layers "*.Cu" "*.Mask") (remove_unused_layers no)
   (roundrect_rratio 0.25) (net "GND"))
  (pad "29" thru_hole circle (at 7.62 16.51 180) (size 1.8 1.8) (drill 1) (layers "*.Cu" "*.Mask") (remove_unused_layers no) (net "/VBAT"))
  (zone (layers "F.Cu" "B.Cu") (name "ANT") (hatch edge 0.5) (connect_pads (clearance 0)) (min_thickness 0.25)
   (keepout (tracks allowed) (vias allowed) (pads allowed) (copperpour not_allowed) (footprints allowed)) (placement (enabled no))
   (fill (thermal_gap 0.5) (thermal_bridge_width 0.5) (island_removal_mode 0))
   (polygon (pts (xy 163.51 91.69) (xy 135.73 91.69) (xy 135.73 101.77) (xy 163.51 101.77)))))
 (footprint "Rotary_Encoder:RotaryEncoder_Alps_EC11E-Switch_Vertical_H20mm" (layer "B.Cu") (at 157.5 106 180)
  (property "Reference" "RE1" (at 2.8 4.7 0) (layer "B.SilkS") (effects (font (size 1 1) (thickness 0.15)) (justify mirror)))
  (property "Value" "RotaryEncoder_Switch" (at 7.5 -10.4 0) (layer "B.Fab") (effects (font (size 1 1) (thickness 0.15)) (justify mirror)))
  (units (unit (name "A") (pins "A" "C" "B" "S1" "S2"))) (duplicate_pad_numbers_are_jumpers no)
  (pad "A" thru_hole rect (at 0 0 180) (size 2 2) (drill 1) (layers "*.Cu" "*.Mask") (remove_unused_layers no) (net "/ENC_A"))
  (pad "B" thru_hole circle (at 0 -5 180) (size 2 2) (drill 1) (layers "*.Cu" "*.Mask") (remove_unused_layers no) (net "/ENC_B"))
  (pad "C" thru_hole circle (at 0 -2.5 180) (size 2 2) (drill 1) (layers "*.Cu" "*.Mask") (remove_unused_layers no) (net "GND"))
  (pad "MP" thru_hole rect (at 7.5 -8.1 180) (size 3.2 2) (drill oval 2.8 1.5) (layers "*.Cu" "*.Mask") (remove_unused_layers no))
  (pad "MP" thru_hole rect (at 7.5 3.1 180) (size 3.2 2) (drill oval 2.8 1.5) (layers "*.Cu" "*.Mask") (remove_unused_layers no))
  (pad "S1" thru_hole circle (at 14.5 -5 180) (size 2 2) (drill 1) (layers "*.Cu" "*.Mask") (remove_unused_layers no) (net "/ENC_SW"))
  (pad "S2" thru_hole circle (at 14.5 0 180) (size 2 2) (drill 1) (layers "*.Cu" "*.Mask") (remove_unused_layers no) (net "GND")))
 (gr_arc (start 126 71.839744) (mid 150 63) (end 174 71.839744) (stroke (width 0.15) (type default)) (layer "Edge.Cuts"))
 (gr_line (start 126 128.160255) (end 126 71.839744) (stroke (width 0.15) (type default)) (layer "Edge.Cuts"))
 (gr_line (start 174 71.839744) (end 174 128.160255) (stroke (width 0.15) (type default)) (layer "Edge.Cuts"))
 (gr_arc (start 174 128.160255) (mid 150 137) (end 126 128.160255) (stroke (width 0.15) (type default)) (layer "Edge.Cuts"))
 (segment (start 132.588 68.961) (end 128.397 73.152) (width 0.4) (layer "F.Cu") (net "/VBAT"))
 (segment (start 142.38 68.03) (end 141.449 68.961) (width 0.4) (layer "F.Cu") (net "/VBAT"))
 (segment (start 128.397 73.152) (end 128.397 91.8) (width 0.4) (layer "F.Cu") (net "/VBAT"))
 (segment (start 128.397 91.8) (end 133.641 97.044) (width 0.4) (layer "F.Cu") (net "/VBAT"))
 (segment (start 142.38 68.03) (end 141.449 68.961) (width 0.4) (layer "F.Cu") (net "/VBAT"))
 (segment (start 141.449 68.961) (end 132.588 68.961) (width 0.4) (layer "F.Cu") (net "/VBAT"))
 (segment (start 128.397 73.152) (end 128.397 91.8) (width 0.4) (layer "F.Cu") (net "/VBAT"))
 (segment (start 128.397 91.8) (end 133.641 97.044) (width 0.4) (layer "F.Cu") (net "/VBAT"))
 (segment (start 132.588 68.961) (end 128.397 73.152) (width 0.4) (layer "F.Cu") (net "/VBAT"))
 (segment (start 142.38 65.49) (end 142.38 68.03) (width 0.4) (layer "F.Cu") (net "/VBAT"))
 (segment (start 164.169 90.89) (end 164.338 91.059) (width 0.25) (layer "F.Cu") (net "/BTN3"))
 (segment (start 157.62 90.89) (end 164.169 90.89) (width 0.25) (layer "F.Cu") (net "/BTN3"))
 (via (at 164.338 91.059) (size 0.6) (drill 0.3) (layers "F.Cu" "B.Cu") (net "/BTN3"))
 (segment (start 170.25 99.638) (end 164.338 93.726) (width 0.25) (layer "B.Cu") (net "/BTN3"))
 (segment (start 170.25 113) (end 170.25 99.638) (width 0.25) (layer "B.Cu") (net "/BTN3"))
 (segment (start 164.338 93.726) (end 164.338 91.059) (width 0.25) (layer "B.Cu") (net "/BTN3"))
 (segment (start 170.25 99.638) (end 164.338 93.726) (width 0.25) (layer "B.Cu") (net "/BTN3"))
 (segment (start 170.25 113) (end 163.75 113) (width 0.25) (layer "B.Cu") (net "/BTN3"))
 (segment (start 164.338 93.726) (end 164.338 91.059) (width 0.25) (layer "B.Cu") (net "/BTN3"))
 (segment (start 153.25 120) (end 146.75 120) (width 0.25) (layer "B.Cu") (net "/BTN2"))
 (segment (start 153.25 120) (end 146.75 120) (width 0.25) (layer "B.Cu") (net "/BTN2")))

